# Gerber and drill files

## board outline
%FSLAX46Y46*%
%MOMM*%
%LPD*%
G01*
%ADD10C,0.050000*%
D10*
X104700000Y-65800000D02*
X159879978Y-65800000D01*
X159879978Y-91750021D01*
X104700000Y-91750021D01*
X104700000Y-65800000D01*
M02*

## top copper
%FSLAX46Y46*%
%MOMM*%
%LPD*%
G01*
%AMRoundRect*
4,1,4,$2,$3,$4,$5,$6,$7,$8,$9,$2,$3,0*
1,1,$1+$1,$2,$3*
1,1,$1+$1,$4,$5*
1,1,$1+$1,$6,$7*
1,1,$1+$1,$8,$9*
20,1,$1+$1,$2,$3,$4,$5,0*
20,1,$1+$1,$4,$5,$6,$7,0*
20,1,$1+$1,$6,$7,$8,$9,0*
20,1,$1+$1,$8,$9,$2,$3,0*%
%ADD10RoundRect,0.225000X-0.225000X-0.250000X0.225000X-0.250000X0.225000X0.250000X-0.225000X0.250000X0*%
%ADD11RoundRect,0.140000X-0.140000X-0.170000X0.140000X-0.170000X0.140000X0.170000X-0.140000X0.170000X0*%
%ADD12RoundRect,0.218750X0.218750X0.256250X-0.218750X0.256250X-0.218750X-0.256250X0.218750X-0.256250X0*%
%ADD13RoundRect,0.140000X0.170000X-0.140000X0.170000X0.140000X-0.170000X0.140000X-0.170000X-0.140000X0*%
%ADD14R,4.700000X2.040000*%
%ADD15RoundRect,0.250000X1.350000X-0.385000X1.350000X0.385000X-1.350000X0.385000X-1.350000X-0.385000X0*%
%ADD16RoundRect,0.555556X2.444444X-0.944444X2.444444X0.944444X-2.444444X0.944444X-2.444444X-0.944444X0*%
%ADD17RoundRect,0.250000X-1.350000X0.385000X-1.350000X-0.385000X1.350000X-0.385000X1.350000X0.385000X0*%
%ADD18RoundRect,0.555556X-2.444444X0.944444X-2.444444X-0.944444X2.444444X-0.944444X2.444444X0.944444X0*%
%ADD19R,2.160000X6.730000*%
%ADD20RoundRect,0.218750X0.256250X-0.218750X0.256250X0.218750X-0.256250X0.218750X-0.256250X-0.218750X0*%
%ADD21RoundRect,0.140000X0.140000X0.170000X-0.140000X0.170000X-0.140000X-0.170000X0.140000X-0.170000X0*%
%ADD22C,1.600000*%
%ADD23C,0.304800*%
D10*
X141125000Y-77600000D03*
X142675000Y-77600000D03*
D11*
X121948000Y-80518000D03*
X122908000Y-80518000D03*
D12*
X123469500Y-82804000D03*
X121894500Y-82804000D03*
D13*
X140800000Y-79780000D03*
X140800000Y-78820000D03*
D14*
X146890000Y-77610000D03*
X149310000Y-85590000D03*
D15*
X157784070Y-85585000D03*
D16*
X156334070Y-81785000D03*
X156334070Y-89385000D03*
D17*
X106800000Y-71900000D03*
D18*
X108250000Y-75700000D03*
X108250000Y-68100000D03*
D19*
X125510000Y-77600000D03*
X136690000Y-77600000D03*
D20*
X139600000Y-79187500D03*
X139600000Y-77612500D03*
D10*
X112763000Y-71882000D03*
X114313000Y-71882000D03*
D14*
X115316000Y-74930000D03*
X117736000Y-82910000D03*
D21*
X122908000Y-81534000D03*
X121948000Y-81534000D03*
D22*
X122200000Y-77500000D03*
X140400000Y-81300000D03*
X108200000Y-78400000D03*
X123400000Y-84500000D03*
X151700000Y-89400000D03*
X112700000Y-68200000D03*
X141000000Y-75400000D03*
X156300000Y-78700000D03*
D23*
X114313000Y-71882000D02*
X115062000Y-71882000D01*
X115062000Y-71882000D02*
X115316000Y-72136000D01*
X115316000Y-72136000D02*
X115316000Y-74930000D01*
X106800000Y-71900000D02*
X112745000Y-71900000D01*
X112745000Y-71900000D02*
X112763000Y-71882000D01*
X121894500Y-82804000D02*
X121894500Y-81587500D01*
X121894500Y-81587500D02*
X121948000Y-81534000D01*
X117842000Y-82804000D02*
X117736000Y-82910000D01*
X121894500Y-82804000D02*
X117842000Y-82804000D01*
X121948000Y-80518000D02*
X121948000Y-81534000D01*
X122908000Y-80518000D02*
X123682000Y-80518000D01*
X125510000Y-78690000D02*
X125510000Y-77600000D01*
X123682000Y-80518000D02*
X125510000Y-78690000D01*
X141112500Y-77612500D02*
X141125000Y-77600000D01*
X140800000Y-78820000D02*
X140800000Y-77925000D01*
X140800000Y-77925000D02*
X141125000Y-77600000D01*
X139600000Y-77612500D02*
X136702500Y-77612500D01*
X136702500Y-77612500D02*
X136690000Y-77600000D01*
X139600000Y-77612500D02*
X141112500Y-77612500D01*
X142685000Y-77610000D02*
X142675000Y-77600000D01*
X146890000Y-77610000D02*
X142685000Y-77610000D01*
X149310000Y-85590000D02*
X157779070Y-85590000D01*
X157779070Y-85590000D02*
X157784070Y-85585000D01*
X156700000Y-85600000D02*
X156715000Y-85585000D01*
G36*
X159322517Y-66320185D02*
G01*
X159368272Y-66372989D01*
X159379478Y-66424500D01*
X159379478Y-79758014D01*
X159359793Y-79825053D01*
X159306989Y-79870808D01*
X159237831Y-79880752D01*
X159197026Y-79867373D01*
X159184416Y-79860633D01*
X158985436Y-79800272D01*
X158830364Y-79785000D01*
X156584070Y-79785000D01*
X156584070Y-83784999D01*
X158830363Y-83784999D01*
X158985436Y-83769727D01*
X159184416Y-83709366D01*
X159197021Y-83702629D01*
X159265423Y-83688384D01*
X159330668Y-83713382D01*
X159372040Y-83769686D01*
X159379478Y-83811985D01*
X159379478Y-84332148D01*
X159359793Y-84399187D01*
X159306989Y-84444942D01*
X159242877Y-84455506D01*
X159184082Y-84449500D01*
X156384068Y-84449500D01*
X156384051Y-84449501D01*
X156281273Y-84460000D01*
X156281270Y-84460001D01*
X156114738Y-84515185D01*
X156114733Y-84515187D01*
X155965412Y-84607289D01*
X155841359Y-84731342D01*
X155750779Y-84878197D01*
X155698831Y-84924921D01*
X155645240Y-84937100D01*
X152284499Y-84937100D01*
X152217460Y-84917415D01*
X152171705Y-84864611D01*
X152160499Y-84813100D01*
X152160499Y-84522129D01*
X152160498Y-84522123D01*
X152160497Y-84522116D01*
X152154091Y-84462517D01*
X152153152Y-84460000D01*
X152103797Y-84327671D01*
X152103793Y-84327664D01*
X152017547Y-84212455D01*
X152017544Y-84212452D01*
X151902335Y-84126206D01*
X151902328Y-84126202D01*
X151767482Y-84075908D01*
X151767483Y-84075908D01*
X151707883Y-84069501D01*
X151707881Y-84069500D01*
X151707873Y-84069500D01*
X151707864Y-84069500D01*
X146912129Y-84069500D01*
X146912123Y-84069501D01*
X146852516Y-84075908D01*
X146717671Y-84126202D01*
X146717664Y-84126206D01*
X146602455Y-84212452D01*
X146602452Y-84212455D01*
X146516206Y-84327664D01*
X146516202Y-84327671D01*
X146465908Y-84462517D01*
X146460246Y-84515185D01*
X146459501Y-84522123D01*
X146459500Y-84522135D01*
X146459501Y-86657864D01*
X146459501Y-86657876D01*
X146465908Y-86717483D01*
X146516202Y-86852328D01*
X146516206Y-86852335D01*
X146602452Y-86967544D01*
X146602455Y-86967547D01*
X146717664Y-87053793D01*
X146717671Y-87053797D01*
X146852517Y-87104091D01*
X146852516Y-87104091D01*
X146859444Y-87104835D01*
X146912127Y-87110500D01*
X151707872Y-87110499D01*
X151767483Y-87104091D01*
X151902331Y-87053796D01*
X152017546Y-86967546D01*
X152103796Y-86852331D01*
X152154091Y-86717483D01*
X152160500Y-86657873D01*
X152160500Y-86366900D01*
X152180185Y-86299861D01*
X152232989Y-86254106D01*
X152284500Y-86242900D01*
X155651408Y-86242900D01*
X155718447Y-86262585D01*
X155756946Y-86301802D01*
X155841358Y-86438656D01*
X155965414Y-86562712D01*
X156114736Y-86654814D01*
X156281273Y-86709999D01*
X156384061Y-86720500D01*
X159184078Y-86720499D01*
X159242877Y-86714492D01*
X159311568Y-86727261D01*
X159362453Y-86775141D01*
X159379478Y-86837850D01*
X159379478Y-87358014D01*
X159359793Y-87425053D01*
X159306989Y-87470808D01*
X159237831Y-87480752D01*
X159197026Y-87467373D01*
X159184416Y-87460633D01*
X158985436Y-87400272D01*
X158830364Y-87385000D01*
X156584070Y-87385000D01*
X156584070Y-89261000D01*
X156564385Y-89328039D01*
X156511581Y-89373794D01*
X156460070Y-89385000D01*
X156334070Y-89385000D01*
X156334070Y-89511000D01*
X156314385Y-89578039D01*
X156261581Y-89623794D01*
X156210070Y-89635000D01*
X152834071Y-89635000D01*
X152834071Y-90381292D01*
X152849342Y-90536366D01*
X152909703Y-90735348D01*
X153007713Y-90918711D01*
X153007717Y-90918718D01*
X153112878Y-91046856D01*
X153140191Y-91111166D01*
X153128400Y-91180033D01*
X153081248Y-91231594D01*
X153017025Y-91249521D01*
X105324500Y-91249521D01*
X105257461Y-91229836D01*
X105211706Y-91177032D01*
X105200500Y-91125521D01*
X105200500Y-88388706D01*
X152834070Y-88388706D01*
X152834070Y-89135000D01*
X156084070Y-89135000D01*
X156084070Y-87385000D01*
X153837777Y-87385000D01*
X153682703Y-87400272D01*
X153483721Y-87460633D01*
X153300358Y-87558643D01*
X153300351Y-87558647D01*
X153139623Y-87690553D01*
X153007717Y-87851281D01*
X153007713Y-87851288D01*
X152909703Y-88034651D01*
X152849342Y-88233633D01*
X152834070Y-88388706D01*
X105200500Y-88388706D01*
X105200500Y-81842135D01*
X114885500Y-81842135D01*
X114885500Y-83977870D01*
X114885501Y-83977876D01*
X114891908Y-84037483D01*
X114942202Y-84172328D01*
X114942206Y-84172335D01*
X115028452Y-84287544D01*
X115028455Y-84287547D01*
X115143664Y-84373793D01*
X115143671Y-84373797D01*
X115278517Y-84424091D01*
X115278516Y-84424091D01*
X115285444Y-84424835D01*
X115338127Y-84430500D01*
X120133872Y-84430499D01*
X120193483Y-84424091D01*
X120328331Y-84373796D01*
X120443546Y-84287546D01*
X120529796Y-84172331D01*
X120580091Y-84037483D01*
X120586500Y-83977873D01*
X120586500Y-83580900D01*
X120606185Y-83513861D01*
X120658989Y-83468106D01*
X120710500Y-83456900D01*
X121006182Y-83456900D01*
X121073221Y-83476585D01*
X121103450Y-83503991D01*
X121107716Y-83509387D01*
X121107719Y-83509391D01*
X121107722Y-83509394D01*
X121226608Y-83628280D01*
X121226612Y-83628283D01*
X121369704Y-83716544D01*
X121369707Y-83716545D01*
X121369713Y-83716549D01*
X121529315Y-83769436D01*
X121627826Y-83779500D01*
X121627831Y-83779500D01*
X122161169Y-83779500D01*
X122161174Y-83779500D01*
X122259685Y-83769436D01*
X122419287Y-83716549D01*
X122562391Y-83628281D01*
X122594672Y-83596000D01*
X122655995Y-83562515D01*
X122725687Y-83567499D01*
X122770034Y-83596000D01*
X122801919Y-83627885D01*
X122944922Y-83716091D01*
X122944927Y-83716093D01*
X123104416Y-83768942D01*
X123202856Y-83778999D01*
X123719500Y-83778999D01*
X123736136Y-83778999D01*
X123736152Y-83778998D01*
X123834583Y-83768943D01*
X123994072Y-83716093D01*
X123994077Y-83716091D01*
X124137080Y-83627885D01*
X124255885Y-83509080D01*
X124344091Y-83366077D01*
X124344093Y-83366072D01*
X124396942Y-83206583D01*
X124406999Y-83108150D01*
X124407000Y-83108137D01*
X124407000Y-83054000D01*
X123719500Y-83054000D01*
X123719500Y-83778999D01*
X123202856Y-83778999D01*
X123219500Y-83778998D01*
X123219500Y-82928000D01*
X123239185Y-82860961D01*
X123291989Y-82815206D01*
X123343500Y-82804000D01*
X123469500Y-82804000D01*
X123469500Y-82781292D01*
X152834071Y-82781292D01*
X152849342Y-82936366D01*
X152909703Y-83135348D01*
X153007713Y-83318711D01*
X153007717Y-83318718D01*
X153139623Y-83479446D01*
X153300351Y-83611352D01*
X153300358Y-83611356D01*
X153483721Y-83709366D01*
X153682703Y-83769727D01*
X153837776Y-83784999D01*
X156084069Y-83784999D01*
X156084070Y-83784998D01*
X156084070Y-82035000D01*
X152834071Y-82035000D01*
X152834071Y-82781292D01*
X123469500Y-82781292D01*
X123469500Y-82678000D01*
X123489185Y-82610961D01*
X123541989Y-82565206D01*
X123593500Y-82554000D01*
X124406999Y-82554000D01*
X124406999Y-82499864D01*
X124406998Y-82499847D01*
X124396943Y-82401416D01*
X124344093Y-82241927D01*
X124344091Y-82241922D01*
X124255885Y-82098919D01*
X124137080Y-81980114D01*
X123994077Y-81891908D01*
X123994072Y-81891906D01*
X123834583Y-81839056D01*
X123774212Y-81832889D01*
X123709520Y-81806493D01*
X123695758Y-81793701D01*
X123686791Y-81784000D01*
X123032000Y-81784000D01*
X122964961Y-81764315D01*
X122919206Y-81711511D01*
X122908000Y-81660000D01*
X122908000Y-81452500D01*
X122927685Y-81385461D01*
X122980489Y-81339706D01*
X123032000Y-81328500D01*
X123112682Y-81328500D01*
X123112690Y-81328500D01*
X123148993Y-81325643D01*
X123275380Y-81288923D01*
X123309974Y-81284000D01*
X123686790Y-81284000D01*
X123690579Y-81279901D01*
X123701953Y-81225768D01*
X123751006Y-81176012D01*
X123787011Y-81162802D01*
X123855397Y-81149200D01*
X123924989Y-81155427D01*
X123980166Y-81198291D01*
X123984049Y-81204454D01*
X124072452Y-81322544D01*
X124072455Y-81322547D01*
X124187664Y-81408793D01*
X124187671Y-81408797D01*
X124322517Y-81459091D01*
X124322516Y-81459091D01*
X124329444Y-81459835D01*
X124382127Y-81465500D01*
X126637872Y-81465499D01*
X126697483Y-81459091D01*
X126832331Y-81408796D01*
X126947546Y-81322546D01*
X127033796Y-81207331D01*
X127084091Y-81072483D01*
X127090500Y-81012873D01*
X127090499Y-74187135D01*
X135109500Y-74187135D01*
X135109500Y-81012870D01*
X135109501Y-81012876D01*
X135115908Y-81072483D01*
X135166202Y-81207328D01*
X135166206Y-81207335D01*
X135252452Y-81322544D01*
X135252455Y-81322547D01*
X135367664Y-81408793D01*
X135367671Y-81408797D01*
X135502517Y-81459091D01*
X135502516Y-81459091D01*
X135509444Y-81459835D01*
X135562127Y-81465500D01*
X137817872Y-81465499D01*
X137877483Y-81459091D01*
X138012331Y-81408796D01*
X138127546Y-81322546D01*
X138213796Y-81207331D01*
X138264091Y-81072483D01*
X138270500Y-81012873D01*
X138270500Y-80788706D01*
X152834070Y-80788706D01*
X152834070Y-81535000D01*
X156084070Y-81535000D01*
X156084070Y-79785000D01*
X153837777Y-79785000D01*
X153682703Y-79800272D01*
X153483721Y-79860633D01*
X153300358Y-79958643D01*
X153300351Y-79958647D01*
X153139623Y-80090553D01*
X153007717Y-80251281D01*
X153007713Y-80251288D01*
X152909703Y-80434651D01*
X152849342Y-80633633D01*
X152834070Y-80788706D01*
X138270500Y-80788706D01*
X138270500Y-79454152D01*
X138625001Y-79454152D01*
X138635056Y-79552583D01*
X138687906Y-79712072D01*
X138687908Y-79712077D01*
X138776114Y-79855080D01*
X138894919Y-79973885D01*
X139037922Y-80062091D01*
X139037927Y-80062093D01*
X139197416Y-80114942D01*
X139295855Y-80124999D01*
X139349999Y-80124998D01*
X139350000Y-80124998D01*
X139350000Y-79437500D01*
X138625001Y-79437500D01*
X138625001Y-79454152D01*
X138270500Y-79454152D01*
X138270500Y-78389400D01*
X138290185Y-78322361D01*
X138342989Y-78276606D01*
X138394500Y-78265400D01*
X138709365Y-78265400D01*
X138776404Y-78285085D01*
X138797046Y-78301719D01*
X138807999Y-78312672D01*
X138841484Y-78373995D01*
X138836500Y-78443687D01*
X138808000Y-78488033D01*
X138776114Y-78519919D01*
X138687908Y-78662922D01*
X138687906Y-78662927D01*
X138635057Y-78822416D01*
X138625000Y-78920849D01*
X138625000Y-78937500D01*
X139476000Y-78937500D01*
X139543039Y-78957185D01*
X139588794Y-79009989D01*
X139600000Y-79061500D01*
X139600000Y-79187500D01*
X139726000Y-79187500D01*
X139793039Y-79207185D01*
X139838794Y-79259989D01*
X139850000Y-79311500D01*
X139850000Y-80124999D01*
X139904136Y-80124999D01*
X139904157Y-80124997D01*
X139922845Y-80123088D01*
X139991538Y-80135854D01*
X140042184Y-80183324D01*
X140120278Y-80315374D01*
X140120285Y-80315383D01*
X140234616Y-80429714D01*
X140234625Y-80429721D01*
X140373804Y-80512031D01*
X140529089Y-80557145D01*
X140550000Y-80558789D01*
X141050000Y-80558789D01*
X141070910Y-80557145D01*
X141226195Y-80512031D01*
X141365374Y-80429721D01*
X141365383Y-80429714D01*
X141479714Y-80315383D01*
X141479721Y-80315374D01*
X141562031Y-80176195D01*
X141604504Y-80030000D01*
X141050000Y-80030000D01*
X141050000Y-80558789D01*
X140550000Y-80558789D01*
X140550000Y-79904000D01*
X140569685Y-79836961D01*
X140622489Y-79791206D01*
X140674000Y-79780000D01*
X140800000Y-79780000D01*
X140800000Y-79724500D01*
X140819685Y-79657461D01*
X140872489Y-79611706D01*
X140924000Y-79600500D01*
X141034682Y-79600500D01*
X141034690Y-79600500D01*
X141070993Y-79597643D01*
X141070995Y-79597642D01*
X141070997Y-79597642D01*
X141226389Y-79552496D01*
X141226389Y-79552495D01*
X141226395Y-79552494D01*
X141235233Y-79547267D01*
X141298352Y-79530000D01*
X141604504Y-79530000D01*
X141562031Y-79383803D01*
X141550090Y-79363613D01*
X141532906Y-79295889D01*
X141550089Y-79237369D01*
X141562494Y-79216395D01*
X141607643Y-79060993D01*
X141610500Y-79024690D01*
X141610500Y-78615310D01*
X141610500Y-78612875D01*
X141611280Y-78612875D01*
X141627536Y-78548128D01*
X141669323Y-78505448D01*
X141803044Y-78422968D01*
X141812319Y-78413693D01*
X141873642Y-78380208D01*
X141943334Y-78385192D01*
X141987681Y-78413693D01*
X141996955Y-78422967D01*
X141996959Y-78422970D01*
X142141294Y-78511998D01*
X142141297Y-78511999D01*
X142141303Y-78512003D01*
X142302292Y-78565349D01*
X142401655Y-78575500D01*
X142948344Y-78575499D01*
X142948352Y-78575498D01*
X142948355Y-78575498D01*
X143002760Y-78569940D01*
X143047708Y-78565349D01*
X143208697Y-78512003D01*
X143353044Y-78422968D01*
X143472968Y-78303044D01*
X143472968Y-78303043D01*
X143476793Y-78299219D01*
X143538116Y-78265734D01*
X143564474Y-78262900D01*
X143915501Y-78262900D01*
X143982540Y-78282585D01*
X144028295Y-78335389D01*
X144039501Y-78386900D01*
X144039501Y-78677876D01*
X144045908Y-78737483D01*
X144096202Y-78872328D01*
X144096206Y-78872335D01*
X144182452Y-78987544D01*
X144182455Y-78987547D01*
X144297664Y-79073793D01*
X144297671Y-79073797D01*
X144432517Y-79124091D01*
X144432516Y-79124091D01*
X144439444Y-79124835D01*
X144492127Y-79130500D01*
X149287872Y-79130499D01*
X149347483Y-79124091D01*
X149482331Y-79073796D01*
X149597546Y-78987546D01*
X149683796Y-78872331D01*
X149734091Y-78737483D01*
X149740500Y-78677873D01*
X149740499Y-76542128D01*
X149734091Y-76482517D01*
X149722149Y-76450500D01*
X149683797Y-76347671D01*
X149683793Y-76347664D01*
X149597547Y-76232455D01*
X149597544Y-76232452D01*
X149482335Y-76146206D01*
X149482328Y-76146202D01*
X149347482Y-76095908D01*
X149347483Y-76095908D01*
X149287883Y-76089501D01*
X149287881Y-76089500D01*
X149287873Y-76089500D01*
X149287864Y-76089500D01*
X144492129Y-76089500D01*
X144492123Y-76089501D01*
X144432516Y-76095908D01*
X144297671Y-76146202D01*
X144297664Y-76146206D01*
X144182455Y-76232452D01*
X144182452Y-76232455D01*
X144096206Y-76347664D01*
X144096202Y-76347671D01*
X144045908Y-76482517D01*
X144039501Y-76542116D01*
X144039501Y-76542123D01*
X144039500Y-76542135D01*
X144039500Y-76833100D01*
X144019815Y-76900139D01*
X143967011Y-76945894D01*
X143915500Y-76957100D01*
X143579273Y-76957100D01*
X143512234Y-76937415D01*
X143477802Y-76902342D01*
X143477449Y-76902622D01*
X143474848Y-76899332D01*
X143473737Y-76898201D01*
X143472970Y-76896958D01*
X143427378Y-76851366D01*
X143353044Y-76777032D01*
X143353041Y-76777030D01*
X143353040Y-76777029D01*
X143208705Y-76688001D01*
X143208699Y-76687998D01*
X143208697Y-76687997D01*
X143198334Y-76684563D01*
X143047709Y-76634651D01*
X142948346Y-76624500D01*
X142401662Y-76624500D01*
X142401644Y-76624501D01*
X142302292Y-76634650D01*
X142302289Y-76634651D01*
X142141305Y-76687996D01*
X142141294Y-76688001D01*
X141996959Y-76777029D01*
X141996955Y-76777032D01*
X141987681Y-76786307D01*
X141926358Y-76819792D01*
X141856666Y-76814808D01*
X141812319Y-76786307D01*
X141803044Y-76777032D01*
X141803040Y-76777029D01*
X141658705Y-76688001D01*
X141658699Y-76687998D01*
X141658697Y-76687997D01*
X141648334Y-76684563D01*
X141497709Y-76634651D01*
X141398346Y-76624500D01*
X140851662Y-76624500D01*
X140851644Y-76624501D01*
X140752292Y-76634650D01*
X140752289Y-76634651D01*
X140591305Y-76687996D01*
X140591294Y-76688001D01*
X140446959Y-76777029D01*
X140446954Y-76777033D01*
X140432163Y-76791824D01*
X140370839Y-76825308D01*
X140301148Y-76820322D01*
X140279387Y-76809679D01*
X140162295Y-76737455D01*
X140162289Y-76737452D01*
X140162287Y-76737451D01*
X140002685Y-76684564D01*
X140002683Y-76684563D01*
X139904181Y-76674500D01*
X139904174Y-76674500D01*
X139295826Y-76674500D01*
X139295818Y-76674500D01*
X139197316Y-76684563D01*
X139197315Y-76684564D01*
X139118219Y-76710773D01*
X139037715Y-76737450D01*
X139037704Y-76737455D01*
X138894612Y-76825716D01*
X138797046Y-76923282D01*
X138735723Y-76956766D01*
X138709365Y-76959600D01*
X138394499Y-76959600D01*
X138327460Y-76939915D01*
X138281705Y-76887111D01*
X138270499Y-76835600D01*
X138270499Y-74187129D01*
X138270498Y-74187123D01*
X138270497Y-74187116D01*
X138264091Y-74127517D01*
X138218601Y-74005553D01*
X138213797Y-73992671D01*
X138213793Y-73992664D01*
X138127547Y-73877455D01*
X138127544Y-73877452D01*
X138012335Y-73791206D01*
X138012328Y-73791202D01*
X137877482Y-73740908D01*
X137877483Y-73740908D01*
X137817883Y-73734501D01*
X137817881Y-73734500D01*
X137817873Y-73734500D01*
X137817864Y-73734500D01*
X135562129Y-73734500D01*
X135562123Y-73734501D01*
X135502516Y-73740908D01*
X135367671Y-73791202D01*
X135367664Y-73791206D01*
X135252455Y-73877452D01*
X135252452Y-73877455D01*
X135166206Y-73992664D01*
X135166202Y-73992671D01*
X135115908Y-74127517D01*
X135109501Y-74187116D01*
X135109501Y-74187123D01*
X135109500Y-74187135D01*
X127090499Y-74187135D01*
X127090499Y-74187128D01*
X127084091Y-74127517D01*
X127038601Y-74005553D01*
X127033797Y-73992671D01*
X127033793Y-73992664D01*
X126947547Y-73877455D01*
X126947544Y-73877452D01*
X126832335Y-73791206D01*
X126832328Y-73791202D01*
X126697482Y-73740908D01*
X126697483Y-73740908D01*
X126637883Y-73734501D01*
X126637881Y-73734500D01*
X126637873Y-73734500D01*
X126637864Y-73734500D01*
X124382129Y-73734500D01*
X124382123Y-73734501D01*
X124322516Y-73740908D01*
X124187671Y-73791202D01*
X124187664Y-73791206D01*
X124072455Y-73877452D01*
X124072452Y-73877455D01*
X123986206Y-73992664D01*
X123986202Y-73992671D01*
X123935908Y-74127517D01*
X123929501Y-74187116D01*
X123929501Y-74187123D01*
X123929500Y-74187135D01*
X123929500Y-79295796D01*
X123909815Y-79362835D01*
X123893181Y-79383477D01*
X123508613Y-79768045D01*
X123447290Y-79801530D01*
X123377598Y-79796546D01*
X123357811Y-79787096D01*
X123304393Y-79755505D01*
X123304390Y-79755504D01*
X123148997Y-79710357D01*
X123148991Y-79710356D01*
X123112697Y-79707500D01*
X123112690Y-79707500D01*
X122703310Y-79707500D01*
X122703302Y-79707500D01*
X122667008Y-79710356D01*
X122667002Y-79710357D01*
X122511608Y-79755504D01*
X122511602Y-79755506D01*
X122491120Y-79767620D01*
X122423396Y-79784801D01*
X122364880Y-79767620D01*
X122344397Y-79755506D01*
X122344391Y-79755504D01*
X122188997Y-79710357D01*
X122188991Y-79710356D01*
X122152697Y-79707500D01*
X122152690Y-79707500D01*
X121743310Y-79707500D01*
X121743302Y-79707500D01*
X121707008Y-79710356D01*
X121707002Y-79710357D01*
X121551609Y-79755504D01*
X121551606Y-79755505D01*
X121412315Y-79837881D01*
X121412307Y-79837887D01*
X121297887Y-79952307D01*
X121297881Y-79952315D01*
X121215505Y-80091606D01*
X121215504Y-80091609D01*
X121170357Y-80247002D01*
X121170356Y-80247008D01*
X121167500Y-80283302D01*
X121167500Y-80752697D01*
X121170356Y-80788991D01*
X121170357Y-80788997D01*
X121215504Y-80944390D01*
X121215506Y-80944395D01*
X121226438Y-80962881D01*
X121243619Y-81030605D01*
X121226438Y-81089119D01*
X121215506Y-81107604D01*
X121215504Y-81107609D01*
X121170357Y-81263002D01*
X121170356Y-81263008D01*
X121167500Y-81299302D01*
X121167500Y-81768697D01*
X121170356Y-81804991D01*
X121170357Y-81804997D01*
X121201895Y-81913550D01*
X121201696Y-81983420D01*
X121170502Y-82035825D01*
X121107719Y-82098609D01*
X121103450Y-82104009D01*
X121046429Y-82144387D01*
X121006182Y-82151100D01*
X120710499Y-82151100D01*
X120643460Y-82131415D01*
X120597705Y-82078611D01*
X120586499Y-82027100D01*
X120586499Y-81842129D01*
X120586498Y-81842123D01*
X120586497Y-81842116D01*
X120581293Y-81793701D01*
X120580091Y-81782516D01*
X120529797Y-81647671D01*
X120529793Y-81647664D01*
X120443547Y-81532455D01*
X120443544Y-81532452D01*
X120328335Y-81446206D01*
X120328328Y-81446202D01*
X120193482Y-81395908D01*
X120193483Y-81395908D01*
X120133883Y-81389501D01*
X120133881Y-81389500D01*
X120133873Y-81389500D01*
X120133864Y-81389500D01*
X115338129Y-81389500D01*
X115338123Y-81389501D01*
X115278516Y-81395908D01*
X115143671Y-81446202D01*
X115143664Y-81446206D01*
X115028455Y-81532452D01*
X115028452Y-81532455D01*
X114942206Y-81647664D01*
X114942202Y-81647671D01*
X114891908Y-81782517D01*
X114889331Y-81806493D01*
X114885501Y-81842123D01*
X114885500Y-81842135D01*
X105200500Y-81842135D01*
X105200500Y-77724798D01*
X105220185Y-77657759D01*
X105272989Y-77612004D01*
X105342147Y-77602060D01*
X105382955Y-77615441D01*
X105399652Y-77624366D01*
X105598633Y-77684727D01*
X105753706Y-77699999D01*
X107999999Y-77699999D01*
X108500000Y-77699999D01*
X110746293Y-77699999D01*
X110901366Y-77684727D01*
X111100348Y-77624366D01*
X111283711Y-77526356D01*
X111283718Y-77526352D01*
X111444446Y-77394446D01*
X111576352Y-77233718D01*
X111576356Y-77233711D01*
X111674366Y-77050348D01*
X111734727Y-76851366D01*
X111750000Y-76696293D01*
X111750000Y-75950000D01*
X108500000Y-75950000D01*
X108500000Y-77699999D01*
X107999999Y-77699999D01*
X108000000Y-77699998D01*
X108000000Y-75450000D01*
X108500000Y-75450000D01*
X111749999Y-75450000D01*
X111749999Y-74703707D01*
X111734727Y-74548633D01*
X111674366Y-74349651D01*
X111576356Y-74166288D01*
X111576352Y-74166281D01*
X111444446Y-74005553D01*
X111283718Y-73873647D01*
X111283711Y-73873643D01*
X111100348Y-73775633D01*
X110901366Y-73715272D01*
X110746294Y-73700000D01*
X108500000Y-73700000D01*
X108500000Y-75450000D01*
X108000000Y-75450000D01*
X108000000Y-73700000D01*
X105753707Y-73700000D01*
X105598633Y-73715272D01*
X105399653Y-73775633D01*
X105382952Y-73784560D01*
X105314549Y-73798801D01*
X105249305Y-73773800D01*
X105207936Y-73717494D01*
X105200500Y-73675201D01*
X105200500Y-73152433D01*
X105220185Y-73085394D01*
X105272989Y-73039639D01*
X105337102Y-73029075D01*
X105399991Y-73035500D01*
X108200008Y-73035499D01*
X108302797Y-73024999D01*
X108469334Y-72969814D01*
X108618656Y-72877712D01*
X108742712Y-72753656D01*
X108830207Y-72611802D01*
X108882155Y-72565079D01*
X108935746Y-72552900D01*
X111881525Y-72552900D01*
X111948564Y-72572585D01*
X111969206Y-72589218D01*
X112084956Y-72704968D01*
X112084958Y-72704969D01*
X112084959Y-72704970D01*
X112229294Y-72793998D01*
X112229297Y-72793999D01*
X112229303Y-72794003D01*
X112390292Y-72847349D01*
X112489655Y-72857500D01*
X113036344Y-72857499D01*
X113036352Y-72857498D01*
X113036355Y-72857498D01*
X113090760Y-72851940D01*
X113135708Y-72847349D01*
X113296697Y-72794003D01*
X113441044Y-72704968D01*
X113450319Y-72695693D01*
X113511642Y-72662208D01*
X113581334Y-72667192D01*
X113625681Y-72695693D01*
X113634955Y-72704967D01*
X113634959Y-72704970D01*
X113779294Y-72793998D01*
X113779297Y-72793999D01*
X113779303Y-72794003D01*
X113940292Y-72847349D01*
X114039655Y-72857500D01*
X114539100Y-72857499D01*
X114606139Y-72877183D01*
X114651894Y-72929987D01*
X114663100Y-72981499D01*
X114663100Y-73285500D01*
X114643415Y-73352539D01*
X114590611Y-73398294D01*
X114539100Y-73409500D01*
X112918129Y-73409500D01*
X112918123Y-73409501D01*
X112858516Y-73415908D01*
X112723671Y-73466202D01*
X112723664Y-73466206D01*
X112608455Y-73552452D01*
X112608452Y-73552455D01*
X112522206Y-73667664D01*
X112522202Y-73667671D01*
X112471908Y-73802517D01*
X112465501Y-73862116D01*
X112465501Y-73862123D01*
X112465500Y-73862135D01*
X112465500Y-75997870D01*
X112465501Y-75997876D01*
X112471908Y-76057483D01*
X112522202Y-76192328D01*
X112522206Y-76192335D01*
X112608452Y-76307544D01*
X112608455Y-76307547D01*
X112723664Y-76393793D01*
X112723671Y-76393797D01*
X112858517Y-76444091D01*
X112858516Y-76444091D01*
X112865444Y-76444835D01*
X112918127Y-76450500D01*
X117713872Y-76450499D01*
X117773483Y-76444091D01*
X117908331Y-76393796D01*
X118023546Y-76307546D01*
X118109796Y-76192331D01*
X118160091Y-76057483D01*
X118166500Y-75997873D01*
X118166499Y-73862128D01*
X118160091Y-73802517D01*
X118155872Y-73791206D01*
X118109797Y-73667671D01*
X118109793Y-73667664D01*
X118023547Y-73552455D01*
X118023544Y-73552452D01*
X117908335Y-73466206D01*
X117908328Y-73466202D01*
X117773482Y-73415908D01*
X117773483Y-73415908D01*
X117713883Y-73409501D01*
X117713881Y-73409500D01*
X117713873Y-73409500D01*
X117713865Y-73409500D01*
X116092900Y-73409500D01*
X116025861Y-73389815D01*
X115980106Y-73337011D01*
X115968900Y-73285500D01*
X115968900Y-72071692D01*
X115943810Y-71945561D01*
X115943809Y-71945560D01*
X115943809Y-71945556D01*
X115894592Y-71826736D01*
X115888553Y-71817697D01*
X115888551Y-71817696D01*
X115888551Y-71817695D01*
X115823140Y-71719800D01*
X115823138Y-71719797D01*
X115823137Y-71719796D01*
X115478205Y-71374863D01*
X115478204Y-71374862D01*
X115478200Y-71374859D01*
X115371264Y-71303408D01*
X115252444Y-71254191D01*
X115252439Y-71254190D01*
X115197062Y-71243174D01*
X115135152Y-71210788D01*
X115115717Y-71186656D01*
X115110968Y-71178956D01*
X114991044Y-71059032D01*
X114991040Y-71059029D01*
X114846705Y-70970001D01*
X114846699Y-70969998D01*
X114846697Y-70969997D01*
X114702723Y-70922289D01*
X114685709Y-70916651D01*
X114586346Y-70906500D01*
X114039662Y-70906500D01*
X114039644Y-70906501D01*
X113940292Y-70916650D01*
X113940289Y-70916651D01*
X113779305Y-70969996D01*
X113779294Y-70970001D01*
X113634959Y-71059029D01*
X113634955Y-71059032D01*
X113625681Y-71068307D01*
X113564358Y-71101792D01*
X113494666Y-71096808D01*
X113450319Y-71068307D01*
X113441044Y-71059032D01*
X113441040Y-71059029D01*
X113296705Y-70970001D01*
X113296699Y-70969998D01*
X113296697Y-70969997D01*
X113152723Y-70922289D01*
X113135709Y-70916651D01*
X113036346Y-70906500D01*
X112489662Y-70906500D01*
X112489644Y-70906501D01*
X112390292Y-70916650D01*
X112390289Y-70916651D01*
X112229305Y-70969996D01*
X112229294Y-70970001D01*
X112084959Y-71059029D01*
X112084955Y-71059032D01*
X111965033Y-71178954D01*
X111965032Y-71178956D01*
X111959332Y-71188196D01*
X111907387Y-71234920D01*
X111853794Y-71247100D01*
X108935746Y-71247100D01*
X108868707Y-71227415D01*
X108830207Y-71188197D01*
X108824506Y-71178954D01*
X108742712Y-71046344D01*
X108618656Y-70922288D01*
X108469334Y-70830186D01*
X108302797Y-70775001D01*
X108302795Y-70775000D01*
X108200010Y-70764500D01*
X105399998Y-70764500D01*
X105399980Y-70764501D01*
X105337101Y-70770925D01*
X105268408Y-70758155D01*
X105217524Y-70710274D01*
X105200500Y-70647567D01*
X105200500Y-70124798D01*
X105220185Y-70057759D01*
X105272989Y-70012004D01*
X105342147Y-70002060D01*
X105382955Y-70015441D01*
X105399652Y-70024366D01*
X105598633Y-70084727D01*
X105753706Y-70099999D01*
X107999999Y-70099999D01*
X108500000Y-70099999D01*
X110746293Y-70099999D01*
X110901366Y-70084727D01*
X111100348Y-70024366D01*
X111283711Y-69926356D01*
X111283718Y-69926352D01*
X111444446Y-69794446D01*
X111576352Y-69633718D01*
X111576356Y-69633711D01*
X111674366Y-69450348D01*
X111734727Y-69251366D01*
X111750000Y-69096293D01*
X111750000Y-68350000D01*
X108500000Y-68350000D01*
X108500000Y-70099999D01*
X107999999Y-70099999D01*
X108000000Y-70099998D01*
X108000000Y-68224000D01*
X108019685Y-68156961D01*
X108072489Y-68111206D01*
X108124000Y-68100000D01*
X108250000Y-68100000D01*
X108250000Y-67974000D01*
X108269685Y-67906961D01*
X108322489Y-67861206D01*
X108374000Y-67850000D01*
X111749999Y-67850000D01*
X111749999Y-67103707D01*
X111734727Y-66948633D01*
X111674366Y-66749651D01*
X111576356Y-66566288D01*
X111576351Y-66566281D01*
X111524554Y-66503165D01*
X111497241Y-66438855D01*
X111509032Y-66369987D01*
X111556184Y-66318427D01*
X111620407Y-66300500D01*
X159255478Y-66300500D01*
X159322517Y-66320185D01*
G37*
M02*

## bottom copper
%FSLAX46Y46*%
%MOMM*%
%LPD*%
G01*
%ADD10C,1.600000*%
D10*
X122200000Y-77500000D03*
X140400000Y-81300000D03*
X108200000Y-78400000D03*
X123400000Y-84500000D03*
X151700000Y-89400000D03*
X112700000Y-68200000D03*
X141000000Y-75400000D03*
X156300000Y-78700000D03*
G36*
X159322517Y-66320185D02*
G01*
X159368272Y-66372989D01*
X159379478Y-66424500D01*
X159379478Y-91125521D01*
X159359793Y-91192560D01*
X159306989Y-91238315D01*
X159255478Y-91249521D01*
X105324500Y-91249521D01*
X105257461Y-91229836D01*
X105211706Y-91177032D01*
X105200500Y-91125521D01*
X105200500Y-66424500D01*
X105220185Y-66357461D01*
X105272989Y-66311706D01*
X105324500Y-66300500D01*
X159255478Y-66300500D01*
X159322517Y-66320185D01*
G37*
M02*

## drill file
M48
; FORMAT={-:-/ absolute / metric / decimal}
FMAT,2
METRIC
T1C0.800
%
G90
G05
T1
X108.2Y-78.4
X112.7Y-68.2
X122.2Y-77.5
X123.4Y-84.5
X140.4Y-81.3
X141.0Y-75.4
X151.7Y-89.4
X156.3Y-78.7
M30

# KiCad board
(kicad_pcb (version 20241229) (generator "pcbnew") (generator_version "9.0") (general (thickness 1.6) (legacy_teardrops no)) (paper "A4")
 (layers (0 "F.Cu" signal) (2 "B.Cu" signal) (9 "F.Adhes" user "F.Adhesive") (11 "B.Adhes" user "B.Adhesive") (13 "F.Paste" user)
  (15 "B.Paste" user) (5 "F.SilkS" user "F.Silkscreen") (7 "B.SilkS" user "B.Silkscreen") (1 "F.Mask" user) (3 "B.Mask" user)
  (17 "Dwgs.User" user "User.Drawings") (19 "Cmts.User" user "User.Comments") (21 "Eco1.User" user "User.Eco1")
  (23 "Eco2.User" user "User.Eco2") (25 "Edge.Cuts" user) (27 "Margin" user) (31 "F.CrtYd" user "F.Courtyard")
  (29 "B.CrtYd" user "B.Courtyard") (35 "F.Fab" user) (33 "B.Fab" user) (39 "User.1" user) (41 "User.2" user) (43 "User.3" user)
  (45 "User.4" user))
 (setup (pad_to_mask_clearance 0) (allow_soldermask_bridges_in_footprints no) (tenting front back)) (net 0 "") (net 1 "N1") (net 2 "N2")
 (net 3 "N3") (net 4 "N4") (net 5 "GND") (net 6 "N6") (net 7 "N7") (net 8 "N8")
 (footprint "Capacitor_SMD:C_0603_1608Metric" (layer "F.Cu") (at 141.9 77.6)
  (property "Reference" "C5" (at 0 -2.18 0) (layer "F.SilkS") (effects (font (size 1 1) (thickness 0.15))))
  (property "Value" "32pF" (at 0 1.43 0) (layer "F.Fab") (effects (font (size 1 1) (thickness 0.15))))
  (pad "1" smd roundrect (at -0.775 0) (size 0.9 0.95) (layers "F.Cu" "F.Mask" "F.Paste") (roundrect_rratio 0.25) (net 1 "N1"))
  (pad "2" smd roundrect (at 0.775 0) (size 0.9 0.95) (layers "F.Cu" "F.Mask" "F.Paste") (roundrect_rratio 0.25) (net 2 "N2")))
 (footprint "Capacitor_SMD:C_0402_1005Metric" (layer "F.Cu") (at 122.428 80.518)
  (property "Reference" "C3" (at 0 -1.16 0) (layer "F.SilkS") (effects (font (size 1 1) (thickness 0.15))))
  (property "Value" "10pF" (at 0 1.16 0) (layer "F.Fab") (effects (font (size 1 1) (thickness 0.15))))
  (pad "1" smd roundrect (at -0.48 0) (size 0.56 0.62) (layers "F.Cu" "F.Mask" "F.Paste") (roundrect_rratio 0.25) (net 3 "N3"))
  (pad "2" smd roundrect (at 0.48 0) (size 0.56 0.62) (layers "F.Cu" "F.Mask" "F.Paste") (roundrect_rratio 0.25) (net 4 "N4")))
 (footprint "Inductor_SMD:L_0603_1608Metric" (layer "F.Cu") (at 122.682 82.804 180)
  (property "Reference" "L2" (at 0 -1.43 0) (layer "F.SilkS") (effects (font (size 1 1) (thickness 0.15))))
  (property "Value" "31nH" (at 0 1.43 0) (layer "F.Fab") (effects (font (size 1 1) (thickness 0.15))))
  (pad "1" smd roundrect (at -0.7875 0 180) (size 0.875 0.95) (layers "F.Cu" "F.Mask" "F.Paste") (roundrect_rratio 0.25) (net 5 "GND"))
  (pad "2" smd roundrect (at 0.7875 0 180) (size 0.875 0.95) (layers "F.Cu" "F.Mask" "F.Paste") (roundrect_rratio 0.25) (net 3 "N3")))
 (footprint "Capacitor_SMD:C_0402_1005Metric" (layer "F.Cu") (at 140.8 79.3 90)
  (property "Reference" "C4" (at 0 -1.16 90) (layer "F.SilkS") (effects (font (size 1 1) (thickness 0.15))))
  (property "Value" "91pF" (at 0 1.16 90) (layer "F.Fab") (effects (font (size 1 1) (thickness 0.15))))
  (pad "1" smd roundrect (at -0.48 0 90) (size 0.56 0.62) (layers "F.Cu" "F.Mask" "F.Paste") (roundrect_rratio 0.25) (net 5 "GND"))
  (pad "2" smd roundrect (at 0.48 0 90) (size 0.56 0.62) (layers "F.Cu" "F.Mask" "F.Paste") (roundrect_rratio 0.25) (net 1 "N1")))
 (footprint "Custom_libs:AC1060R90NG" (layer "F.Cu") (at 148.1 81.6 -90)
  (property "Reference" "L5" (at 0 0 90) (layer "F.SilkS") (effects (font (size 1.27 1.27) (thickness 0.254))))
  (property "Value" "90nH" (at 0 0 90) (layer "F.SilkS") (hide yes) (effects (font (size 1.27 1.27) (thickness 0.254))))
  (pad "1" smd rect (at -3.99 1.21 270) (size 2.04 4.7) (layers "F.Cu" "F.Mask" "F.Paste") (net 2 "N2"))
  (pad "2" smd rect (at 3.99 -1.21 270) (size 2.04 4.7) (layers "F.Cu" "F.Mask" "F.Paste") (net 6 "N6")))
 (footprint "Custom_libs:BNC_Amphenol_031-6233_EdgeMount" (layer "F.Cu") (at 157.78407 85.585)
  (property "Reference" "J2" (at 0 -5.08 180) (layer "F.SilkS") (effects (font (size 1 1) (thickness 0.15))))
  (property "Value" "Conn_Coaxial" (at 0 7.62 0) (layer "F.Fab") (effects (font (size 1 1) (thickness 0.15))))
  (pad "1" smd roundrect (at 0 0 90) (size 1.27 3.2) (layers "F.Cu" "F.Mask") (roundrect_rratio 0.1968503937) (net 6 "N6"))
  (pad "2" smd roundrect (at -1.45 -3.8 90) (size 3 6) (layers "F.Cu" "F.Mask") (roundrect_rratio 0.1851851852) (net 5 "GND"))
  (pad "2" smd roundrect (at -1.45 3.8 90) (size 3 6) (layers "F.Cu" "F.Mask") (roundrect_rratio 0.1851851852) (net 5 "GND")))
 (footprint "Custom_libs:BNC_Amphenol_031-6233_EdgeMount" (layer "F.Cu") (at 106.8 71.9 180)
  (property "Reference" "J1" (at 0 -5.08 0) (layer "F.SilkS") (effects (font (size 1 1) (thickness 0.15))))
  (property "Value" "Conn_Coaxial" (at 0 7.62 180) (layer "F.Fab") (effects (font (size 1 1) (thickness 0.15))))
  (pad "1" smd roundrect (at 0 0 270) (size 1.27 3.2) (layers "F.Cu" "F.Mask") (roundrect_rratio 0.1968503937) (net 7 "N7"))
  (pad "2" smd roundrect (at -1.45 -3.8 270) (size 3 6) (layers "F.Cu" "F.Mask") (roundrect_rratio 0.1851851852) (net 5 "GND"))
  (pad "2" smd roundrect (at -1.45 3.8 270) (size 3 6) (layers "F.Cu" "F.Mask") (roundrect_rratio 0.1851851852) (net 5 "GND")))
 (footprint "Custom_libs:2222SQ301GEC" (layer "F.Cu") (at 131.1 77.6)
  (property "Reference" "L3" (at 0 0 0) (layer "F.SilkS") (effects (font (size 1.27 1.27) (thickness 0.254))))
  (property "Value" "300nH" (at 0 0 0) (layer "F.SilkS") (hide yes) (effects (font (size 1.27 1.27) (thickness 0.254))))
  (pad "1" smd rect (at -5.59 0) (size 2.16 6.73) (layers "F.Cu" "F.Mask" "F.Paste") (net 4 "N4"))
  (pad "2" smd rect (at 5.59 0) (size 2.16 6.73) (layers "F.Cu" "F.Mask" "F.Paste") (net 1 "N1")))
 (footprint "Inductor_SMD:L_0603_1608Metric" (layer "F.Cu") (at 139.6 78.4 90)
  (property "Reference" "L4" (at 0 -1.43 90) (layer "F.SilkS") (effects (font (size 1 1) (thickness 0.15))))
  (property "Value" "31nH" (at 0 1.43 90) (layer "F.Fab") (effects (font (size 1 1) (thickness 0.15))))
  (pad "1" smd roundrect (at -0.7875 0 90) (size 0.875 0.95) (layers "F.Cu" "F.Mask" "F.Paste") (roundrect_rratio 0.25) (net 5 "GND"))
  (pad "2" smd roundrect (at 0.7875 0 90) (size 0.875 0.95) (layers "F.Cu" "F.Mask" "F.Paste") (roundrect_rratio 0.25) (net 1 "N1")))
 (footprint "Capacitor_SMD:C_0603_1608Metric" (layer "F.Cu") (at 113.538 71.882)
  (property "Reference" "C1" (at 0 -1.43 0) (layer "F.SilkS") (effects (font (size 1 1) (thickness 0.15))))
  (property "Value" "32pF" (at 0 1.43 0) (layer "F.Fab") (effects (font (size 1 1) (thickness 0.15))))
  (pad "1" smd roundrect (at -0.775 0) (size 0.9 0.95) (layers "F.Cu" "F.Mask" "F.Paste") (roundrect_rratio 0.25) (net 7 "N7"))
  (pad "2" smd roundrect (at 0.775 0) (size 0.9 0.95) (layers "F.Cu" "F.Mask" "F.Paste") (roundrect_rratio 0.25) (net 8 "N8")))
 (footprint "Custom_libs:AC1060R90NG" (layer "F.Cu") (at 116.526 78.92 -90)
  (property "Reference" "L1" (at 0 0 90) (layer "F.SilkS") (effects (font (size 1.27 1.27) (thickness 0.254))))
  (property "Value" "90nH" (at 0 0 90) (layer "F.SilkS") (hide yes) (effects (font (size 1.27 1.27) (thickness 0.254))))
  (pad "1" smd rect (at -3.99 1.21 270) (size 2.04 4.7) (layers "F.Cu" "F.Mask" "F.Paste") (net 8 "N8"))
  (pad "2" smd rect (at 3.99 -1.21 270) (size 2.04 4.7) (layers "F.Cu" "F.Mask" "F.Paste") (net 3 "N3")))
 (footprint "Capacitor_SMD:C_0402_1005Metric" (layer "F.Cu") (at 122.428 81.534 180)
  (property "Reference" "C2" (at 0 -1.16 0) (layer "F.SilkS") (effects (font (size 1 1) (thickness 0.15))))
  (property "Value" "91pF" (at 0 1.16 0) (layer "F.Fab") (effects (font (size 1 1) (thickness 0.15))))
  (pad "1" smd roundrect (at -0.48 0 180) (size 0.56 0.62) (layers "F.Cu" "F.Mask" "F.Paste") (roundrect_rratio 0.25) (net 5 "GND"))
  (pad "2" smd roundrect (at 0.48 0 180) (size 0.56 0.62) (layers "F.Cu" "F.Mask" "F.Paste") (roundrect_rratio 0.25) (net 3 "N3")))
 (gr_rect (start 104.7 65.8) (end 159.879978 91.750021) (stroke (width 0.05) (type solid)) (fill no) (layer "Edge.Cuts"))
 (segment (start 114.313 71.882) (end 115.062 71.882) (width 0.3048) (layer "F.Cu") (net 8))
 (segment (start 115.062 71.882) (end 115.316 72.136) (width 0.3048) (layer "F.Cu") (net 8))
 (segment (start 115.316 72.136) (end 115.316 74.93) (width 0.3048) (layer "F.Cu") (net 8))
 (segment (start 106.8 71.9) (end 112.745 71.9) (width 0.3048) (layer "F.Cu") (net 7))
 (segment (start 112.745 71.9) (end 112.763 71.882) (width 0.3048) (layer "F.Cu") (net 7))
 (via (at 122.2 77.5) (size 1.6) (drill 0.8) (layers "F.Cu" "B.Cu") (free yes) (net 5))
 (via (at 140.4 81.3) (size 1.6) (drill 0.8) (layers "F.Cu" "B.Cu") (free yes) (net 5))
 (via (at 108.2 78.4) (size 1.6) (drill 0.8) (layers "F.Cu" "B.Cu") (free yes) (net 5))
 (via (at 123.4 84.5) (size 1.6) (drill 0.8) (layers "F.Cu" "B.Cu") (free yes) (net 5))
 (via (at 151.7 89.4) (size 1.6) (drill 0.8) (layers "F.Cu" "B.Cu") (free yes) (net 5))
 (via (at 112.7 68.2) (size 1.6) (drill 0.8) (layers "F.Cu" "B.Cu") (free yes) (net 5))
 (via (at 141 75.4) (size 1.6) (drill 0.8) (layers "F.Cu" "B.Cu") (free yes) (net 5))
 (via (at 156.3 78.7) (size 1.6) (drill 0.8) (layers "F.Cu" "B.Cu") (free yes) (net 5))
 (segment (start 121.8945 82.804) (end 121.8945 81.5875) (width 0.3048) (layer "F.Cu") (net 3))
 (segment (start 121.8945 81.5875) (end 121.948 81.534) (width 0.3048) (layer "F.Cu") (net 3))
 (segment (start 117.842 82.804) (end 117.736 82.91) (width 0.3048) (layer "F.Cu") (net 3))
 (segment (start 121.8945 82.804) (end 117.842 82.804) (width 0.3048) (layer "F.Cu") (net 3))
 (segment (start 121.948 80.518) (end 121.948 81.534) (width 0.3048) (layer "F.Cu") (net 3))
 (segment (start 122.908 80.518) (end 123.682 80.518) (width 0.3048) (layer "F.Cu") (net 4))
 (segment (start 125.51 78.69) (end 125.51 77.6) (width 0.3048) (layer "F.Cu") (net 4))
 (segment (start 123.682 80.518) (end 125.51 78.69) (width 0.3048) (layer "F.Cu") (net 4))
 (segment (start 141.1125 77.6125) (end 141.125 77.6) (width 0.3048) (layer "F.Cu") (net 1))
 (segment (start 140.8 78.82) (end 140.8 77.925) (width 0.3048) (layer "F.Cu") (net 1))
 (segment (start 140.8 77.925) (end 141.125 77.6) (width 0.3048) (layer "F.Cu") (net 1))
 (segment (start 139.6 77.6125) (end 136.7025 77.6125) (width 0.3048) (layer "F.Cu") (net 1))
 (segment (start 136.7025 77.6125) (end 136.69 77.6) (width 0.3048) (layer "F.Cu") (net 1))
 (segment (start 139.6 77.6125) (end 141.1125 77.6125) (width 0.3048) (layer "F.Cu") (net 1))
 (segment (start 142.685 77.61) (end 142.675 77.6) (width 0.3048) (layer "F.Cu") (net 2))
 (segment (start 146.89 77.61) (end 142.685 77.61) (width 0.3048) (layer "F.Cu") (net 2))
 (segment (start 149.31 85.59) (end 157.77907 85.59) (width 0.3048) (layer "F.Cu") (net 6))
 (segment (start 157.77907 85.59) (end 157.78407 85.585) (width 0.3048) (layer "F.Cu") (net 6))
 (segment (start 156.7 85.6) (end 156.715 85.585) (width 0.3048) (layer "F.Cu") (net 6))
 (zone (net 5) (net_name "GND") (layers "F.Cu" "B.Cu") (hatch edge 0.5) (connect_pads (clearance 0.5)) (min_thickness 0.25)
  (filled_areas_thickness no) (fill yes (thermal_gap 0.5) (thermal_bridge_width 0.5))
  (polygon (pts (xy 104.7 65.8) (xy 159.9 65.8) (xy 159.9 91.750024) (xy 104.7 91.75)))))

